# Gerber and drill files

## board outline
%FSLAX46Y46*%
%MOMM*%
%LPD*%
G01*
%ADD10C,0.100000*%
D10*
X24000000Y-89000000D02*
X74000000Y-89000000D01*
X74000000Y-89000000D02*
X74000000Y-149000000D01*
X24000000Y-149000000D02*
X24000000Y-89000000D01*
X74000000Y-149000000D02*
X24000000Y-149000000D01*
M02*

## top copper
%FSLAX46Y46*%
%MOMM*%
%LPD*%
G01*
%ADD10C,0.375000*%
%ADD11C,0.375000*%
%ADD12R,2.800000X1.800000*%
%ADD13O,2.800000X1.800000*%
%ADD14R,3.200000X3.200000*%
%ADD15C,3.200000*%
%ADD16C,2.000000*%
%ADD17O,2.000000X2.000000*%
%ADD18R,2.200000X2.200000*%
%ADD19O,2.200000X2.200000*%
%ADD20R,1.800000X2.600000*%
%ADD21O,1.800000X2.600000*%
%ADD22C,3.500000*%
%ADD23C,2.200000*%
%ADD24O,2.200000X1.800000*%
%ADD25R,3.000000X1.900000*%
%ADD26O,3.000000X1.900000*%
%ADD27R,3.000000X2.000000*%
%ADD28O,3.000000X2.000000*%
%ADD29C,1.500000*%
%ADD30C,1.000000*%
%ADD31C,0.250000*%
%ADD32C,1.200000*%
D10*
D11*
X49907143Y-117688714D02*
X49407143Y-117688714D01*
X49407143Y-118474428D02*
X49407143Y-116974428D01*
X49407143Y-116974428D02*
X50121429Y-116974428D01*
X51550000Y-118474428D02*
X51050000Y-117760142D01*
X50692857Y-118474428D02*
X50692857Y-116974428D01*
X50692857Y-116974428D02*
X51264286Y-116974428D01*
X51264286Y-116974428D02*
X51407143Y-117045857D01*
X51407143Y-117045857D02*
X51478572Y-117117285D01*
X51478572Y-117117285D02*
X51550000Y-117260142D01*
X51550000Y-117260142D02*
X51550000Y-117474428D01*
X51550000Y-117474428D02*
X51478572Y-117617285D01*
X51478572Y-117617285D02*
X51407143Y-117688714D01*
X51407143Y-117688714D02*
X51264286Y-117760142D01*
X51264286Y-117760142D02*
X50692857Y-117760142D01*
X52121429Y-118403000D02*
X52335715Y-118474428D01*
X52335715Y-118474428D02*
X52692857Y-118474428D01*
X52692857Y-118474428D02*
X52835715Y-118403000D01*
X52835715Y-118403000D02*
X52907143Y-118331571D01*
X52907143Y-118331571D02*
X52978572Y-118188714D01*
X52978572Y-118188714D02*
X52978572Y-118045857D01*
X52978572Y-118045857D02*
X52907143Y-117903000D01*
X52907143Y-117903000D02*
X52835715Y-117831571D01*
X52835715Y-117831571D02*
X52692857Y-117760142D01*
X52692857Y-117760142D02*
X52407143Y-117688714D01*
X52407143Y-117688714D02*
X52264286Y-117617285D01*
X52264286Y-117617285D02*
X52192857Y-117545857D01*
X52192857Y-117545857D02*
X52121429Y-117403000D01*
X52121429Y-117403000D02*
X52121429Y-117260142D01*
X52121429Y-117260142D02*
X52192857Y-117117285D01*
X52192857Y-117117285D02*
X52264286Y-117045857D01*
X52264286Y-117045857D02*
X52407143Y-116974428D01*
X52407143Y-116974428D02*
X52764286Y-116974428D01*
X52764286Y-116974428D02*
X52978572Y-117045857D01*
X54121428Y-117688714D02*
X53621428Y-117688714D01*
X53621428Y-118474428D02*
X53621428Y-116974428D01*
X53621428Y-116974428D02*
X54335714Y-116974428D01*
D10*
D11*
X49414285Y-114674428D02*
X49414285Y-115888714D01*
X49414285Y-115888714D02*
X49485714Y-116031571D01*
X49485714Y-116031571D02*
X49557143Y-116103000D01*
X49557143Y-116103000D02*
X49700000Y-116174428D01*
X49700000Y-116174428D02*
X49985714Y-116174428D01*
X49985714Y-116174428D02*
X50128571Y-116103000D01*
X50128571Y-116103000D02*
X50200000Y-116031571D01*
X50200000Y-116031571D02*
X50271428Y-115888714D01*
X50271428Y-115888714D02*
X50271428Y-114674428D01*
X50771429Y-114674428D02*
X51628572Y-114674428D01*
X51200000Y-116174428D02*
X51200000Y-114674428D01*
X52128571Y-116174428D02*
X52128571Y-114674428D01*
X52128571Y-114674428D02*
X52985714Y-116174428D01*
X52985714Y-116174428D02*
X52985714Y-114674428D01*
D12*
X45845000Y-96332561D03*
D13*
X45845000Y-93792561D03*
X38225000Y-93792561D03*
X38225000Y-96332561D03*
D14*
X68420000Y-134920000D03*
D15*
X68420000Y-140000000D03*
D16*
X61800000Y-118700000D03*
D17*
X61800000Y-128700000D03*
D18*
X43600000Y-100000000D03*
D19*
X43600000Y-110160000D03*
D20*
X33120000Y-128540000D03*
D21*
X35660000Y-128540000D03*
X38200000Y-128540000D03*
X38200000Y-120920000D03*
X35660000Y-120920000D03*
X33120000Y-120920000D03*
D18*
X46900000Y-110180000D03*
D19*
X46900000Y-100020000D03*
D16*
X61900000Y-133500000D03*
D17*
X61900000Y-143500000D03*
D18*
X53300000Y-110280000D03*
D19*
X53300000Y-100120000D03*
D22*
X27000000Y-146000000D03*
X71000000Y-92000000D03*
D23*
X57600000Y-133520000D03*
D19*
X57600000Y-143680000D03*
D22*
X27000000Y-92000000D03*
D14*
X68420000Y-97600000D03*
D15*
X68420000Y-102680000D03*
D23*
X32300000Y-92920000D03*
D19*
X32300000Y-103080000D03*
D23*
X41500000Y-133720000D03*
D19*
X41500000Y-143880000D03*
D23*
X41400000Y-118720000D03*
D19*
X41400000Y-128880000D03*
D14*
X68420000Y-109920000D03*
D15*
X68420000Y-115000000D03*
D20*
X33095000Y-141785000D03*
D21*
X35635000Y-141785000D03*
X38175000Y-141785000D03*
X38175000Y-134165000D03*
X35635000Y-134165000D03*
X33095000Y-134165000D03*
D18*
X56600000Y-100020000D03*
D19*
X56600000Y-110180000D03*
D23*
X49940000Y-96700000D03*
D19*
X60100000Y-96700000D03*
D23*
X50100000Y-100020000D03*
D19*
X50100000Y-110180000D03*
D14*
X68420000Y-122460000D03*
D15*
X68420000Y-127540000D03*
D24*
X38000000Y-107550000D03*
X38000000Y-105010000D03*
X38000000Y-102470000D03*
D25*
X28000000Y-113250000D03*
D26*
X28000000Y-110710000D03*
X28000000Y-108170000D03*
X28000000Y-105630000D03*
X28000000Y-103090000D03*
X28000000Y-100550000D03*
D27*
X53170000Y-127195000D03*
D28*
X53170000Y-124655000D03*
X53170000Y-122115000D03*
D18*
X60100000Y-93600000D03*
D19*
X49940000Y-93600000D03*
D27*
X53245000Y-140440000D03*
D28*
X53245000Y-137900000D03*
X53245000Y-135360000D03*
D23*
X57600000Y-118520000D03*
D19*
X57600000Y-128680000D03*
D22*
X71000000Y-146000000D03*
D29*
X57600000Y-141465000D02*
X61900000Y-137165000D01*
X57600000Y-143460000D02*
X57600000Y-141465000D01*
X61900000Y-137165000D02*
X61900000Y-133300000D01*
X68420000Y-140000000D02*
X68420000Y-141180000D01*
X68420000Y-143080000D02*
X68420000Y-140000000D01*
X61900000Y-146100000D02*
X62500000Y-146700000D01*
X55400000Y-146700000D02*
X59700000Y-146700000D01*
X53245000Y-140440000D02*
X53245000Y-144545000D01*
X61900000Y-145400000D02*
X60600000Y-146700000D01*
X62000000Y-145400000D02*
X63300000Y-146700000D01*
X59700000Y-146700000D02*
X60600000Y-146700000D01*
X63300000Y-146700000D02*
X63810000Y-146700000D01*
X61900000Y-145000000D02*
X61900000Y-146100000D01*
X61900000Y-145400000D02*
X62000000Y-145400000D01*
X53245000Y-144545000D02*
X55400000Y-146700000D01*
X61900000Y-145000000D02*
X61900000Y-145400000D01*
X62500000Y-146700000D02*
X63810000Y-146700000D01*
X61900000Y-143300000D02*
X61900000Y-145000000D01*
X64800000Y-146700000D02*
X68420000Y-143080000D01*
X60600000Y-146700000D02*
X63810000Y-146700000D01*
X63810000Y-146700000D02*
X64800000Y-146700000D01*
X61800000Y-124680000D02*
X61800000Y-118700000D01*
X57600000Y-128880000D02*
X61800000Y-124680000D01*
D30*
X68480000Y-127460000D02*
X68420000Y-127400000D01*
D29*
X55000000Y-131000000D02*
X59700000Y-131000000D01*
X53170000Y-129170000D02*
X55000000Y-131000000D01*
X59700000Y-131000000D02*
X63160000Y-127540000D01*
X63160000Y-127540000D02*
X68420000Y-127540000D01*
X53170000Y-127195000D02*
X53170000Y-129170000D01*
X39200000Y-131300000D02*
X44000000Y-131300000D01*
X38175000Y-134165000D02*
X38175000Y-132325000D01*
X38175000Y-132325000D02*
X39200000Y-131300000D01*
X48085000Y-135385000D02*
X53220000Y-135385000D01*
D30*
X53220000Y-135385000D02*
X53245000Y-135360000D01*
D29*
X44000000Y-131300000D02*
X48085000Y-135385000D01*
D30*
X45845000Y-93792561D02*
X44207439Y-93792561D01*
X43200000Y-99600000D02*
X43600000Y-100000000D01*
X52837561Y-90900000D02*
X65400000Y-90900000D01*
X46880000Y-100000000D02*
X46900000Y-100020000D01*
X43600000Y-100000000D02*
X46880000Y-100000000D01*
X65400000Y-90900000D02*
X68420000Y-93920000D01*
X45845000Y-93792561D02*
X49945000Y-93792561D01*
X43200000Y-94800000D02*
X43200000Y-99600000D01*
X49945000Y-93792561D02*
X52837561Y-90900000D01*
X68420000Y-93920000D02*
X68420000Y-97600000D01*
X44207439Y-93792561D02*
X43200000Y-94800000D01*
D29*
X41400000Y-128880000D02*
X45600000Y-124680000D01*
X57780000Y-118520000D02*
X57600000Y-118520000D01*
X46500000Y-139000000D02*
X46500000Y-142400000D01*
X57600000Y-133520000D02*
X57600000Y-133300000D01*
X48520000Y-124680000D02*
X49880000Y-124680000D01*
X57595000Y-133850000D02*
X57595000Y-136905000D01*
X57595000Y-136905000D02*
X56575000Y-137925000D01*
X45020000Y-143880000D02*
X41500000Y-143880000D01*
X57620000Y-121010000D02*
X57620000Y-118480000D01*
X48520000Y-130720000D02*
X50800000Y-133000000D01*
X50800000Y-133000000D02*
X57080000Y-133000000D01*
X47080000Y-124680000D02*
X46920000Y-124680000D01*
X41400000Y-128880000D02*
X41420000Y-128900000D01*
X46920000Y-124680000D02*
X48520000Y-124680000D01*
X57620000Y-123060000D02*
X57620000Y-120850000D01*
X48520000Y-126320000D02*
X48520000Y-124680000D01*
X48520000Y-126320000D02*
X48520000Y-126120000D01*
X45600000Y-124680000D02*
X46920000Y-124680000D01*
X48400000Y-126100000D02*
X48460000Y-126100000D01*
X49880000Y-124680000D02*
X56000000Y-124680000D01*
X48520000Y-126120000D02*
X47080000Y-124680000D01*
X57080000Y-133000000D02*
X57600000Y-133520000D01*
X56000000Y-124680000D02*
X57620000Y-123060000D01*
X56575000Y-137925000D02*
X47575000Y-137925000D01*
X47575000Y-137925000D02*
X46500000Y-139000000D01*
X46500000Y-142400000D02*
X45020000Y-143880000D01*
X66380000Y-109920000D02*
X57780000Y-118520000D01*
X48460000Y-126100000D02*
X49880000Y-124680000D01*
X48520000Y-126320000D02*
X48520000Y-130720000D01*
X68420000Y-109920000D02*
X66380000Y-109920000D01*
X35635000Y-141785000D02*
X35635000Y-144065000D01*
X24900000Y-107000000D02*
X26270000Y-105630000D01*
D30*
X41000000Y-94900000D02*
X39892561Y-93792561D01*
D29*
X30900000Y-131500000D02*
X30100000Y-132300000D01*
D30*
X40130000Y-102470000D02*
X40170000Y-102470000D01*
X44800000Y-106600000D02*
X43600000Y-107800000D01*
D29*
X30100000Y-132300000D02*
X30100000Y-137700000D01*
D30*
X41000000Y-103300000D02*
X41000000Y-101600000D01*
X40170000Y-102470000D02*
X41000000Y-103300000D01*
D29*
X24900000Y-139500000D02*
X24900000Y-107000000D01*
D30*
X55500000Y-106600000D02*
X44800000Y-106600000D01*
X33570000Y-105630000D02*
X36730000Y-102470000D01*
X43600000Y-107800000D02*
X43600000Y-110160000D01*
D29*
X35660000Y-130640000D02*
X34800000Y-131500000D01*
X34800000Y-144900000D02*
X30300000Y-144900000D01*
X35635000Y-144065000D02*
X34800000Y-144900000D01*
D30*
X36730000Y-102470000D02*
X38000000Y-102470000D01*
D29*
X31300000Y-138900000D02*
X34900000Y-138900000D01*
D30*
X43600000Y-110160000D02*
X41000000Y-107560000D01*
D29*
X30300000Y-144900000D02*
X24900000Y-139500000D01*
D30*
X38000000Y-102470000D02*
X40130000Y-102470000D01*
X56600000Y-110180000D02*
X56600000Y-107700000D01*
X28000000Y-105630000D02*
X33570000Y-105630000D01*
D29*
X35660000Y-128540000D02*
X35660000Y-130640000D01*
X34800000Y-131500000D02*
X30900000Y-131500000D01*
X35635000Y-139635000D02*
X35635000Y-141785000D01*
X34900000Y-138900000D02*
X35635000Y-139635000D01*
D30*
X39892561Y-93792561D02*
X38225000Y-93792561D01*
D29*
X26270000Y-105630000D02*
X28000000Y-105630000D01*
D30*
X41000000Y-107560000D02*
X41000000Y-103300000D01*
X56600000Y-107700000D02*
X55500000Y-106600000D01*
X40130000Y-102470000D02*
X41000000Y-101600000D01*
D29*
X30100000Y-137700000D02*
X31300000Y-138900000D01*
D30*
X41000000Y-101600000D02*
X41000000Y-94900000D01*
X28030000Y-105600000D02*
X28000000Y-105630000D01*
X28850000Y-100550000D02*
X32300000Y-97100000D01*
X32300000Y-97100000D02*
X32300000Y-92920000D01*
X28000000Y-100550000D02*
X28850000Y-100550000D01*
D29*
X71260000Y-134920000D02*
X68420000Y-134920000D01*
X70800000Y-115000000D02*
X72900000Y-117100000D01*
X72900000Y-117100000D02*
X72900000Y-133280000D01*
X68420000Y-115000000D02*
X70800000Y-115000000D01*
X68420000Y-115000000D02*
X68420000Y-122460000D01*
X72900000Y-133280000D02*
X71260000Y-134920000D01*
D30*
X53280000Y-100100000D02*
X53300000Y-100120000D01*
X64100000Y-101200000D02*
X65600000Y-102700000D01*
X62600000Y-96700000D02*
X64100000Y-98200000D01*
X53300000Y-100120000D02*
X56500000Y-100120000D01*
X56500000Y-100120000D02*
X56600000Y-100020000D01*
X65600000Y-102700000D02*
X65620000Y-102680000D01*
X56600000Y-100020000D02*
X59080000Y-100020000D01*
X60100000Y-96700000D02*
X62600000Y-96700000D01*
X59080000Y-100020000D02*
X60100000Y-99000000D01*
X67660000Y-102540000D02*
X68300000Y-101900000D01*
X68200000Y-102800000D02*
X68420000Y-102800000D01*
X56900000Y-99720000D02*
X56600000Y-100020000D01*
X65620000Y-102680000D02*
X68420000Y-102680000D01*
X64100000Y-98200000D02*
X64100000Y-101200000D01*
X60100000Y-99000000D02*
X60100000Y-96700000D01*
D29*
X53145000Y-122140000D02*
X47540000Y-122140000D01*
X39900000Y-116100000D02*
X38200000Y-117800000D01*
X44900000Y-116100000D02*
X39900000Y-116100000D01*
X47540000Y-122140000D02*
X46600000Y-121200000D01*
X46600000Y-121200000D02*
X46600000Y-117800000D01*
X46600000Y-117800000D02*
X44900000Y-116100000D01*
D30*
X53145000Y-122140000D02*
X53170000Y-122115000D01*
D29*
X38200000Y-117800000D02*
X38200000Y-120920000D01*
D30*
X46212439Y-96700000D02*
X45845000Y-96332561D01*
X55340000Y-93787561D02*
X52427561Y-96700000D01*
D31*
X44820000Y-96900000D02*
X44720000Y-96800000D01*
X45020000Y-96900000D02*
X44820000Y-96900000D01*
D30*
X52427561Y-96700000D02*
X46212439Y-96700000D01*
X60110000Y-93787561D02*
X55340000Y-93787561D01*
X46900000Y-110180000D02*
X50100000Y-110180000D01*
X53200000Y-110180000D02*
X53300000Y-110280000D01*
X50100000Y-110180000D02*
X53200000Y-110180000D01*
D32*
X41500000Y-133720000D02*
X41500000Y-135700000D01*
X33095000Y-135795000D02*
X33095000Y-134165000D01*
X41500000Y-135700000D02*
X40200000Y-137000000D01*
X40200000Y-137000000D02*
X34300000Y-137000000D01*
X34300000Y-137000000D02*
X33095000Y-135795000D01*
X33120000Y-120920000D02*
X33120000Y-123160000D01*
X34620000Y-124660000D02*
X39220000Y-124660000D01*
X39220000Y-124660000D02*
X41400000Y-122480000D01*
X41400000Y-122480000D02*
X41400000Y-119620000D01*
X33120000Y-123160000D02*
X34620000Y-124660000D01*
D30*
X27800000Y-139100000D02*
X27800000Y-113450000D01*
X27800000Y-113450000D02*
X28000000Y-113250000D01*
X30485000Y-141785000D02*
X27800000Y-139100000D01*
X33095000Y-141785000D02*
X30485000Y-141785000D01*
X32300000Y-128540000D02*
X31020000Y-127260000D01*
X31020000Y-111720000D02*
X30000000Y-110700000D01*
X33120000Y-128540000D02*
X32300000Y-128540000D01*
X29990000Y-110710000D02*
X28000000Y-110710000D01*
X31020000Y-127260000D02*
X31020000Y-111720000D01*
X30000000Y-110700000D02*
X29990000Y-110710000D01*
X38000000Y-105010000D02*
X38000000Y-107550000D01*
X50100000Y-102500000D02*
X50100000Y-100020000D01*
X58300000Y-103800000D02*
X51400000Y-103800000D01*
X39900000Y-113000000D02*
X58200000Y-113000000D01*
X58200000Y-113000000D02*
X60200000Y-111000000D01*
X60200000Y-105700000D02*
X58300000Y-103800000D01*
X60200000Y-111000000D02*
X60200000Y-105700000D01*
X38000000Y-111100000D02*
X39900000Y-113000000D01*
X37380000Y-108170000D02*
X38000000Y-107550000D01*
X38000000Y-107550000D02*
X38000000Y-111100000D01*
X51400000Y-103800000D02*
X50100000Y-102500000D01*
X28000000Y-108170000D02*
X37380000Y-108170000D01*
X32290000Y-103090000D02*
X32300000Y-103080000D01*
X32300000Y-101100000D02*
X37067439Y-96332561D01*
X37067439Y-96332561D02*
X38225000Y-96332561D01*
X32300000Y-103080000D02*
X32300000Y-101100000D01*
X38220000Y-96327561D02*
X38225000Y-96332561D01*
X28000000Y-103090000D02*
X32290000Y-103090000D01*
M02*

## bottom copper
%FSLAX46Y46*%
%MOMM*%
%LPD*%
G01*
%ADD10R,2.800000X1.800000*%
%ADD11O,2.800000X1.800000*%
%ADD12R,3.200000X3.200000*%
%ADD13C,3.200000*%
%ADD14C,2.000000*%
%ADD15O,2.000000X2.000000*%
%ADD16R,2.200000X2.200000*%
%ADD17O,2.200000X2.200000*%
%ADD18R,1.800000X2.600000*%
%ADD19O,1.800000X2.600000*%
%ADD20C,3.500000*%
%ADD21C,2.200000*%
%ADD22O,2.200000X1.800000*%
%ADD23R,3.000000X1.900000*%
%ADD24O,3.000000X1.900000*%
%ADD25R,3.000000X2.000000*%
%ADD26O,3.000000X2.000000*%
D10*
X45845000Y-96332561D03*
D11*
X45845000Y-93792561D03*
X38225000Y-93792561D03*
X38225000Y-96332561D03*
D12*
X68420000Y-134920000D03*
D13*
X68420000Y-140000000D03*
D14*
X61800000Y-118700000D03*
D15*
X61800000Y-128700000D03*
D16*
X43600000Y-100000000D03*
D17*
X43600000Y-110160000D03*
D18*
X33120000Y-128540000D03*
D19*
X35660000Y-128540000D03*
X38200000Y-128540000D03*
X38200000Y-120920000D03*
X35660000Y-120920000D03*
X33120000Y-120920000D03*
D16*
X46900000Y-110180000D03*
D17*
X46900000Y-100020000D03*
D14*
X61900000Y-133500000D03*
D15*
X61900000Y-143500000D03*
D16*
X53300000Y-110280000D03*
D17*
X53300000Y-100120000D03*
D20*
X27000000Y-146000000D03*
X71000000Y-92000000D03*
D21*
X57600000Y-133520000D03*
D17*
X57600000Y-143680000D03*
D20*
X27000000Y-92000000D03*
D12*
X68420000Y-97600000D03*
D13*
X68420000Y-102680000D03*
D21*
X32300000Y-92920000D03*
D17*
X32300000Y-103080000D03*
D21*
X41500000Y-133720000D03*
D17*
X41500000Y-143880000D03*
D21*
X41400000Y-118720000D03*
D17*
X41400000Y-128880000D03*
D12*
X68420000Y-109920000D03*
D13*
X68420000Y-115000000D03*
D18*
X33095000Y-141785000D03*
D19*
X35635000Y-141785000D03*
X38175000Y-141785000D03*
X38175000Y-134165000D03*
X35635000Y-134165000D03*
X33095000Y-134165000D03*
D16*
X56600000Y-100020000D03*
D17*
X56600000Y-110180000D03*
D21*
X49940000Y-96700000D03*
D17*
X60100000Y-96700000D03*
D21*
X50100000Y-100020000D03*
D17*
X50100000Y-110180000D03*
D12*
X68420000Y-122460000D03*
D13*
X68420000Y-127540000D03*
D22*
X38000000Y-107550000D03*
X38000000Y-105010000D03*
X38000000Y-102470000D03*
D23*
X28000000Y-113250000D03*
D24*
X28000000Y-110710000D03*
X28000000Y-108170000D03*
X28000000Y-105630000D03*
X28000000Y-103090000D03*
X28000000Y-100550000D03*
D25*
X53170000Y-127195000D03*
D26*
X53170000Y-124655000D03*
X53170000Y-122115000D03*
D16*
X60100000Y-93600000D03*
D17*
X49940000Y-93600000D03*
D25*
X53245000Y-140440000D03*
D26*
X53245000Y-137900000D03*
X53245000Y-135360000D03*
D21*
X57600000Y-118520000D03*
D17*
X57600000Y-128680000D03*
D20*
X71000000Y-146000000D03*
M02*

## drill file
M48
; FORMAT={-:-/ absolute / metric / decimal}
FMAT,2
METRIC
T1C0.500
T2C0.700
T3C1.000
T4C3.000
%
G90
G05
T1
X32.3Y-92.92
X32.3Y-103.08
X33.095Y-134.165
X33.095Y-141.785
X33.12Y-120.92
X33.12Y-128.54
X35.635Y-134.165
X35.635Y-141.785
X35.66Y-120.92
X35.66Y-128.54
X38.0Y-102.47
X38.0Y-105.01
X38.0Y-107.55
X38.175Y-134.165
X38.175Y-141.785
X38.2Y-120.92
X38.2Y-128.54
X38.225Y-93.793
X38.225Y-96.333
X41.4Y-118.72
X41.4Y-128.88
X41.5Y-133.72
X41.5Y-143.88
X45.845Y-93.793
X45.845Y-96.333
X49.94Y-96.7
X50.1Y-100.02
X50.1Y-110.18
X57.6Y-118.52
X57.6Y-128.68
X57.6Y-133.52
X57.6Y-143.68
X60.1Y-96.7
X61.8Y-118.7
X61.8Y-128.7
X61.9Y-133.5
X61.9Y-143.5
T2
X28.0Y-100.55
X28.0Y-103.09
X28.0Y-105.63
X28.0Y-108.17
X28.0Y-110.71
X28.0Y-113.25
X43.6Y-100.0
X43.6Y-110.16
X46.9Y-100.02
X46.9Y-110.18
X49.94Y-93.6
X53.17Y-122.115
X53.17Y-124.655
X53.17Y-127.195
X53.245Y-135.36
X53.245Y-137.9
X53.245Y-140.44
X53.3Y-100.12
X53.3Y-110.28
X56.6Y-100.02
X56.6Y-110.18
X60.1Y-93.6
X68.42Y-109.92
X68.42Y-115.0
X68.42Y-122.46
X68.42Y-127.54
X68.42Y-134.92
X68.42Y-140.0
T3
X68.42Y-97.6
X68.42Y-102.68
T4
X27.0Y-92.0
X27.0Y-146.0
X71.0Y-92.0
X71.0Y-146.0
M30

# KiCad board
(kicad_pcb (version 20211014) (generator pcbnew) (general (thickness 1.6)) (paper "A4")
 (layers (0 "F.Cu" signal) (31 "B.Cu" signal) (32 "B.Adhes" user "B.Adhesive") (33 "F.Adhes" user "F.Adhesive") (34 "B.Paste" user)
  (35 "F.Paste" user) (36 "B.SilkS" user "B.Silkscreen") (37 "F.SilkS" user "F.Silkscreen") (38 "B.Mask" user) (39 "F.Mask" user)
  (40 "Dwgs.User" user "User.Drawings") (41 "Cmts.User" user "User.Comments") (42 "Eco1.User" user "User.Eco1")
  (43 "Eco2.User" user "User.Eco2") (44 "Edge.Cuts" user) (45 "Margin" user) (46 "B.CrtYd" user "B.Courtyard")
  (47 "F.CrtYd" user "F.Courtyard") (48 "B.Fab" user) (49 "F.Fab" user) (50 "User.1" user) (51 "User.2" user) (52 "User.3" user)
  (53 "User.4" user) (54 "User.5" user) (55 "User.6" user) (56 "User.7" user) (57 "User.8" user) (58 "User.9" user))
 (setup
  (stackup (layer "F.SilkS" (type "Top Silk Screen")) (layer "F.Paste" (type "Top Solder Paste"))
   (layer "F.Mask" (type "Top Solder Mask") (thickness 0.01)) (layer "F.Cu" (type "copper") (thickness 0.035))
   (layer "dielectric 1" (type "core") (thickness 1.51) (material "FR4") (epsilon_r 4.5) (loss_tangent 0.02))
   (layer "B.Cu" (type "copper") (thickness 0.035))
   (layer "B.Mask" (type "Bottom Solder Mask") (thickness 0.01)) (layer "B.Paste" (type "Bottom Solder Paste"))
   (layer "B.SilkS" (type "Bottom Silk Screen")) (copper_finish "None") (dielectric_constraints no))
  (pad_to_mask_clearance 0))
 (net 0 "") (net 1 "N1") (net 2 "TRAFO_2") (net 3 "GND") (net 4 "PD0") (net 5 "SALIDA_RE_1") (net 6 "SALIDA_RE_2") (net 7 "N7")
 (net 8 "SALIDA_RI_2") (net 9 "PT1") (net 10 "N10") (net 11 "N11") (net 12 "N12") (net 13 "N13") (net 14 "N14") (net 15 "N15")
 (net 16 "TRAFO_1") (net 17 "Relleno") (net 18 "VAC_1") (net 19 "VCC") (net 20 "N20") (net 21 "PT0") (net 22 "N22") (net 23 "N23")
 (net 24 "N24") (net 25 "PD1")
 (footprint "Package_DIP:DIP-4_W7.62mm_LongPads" (layer "F.Cu") (at 45.845 96.332561 180)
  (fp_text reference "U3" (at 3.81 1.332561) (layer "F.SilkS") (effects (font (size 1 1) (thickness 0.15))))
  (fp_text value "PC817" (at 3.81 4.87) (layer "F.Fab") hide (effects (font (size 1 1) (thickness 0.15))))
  (pad "1" thru_hole rect (at 0 0 180) (size 2.8 1.8) (drill 0.5) (layers *.Cu *.Mask) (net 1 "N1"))
  (pad "2" thru_hole oval (at 0 2.54 180) (size 2.8 1.8) (drill 0.5) (layers *.Cu *.Mask) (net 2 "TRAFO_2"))
  (pad "3" thru_hole oval (at 7.62 2.54 180) (size 2.8 1.8) (drill 0.5) (layers *.Cu *.Mask) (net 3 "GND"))
  (pad "4" thru_hole oval (at 7.62 0 180) (size 2.8 1.8) (drill 0.5) (layers *.Cu *.Mask) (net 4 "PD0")))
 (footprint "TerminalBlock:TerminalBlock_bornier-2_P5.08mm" (layer "F.Cu") (at 68.42 134.92 -90)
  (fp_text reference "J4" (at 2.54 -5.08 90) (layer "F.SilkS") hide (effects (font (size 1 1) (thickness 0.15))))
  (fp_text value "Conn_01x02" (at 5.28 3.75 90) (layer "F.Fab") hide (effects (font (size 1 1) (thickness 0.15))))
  (pad "1" thru_hole rect (at 0 0 270) (size 3.2 3.2) (drill 0.7) (layers *.Cu *.Mask) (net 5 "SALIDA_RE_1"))
  (pad "2" thru_hole circle (at 5.08 0 270) (size 3.2 3.2) (drill 0.7) (layers *.Cu *.Mask) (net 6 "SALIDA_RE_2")))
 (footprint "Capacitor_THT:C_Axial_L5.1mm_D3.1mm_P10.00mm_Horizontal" (layer "F.Cu") (at 61.8 118.7 -90)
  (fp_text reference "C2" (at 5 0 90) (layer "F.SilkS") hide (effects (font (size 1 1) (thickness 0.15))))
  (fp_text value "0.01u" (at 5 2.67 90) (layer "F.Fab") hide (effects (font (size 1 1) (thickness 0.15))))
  (pad "1" thru_hole circle (at 0 0 270) (size 2 2) (drill 0.5) (layers *.Cu *.Mask) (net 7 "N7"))
  (pad "2" thru_hole oval (at 10 0 270) (size 2 2) (drill 0.5) (layers *.Cu *.Mask) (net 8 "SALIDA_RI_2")))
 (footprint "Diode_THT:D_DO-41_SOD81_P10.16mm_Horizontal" (layer "F.Cu") (at 43.6 100 -90)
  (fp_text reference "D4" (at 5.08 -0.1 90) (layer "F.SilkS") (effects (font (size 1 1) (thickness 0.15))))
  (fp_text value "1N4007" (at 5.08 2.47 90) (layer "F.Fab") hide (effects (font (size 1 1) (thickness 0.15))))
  (pad "1" thru_hole rect (at 0 0 270) (size 2.2 2.2) (drill 0.7) (layers *.Cu *.Mask) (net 2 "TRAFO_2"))
  (pad "2" thru_hole oval (at 10.16 0 270) (size 2.2 2.2) (drill 0.7) (layers *.Cu *.Mask) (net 3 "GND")))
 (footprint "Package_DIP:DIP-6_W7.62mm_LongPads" (layer "F.Cu") (at 33.12 128.54 90)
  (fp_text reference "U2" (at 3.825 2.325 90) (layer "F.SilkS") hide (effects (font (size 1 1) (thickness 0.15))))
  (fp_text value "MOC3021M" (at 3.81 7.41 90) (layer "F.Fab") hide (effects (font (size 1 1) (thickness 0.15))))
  (pad "1" thru_hole rect (at 0 0 90) (size 2.6 1.8) (drill 0.5) (layers *.Cu *.Mask) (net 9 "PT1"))
  (pad "2" thru_hole oval (at 0 2.54 90) (size 2.6 1.8) (drill 0.5) (layers *.Cu *.Mask) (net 3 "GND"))
  (pad "3" thru_hole oval (at 0 5.08 90) (size 2.6 1.8) (drill 0.5) (layers *.Cu *.Mask) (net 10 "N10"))
  (pad "4" thru_hole oval (at 7.62 5.08 90) (size 2.6 1.8) (drill 0.5) (layers *.Cu *.Mask) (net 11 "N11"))
  (pad "5" thru_hole oval (at 7.62 2.54 90) (size 2.6 1.8) (drill 0.5) (layers *.Cu *.Mask) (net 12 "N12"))
  (pad "6" thru_hole oval (at 7.62 0 90) (size 2.6 1.8) (drill 0.5) (layers *.Cu *.Mask) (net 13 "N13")))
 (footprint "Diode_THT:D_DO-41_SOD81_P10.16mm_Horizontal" (layer "F.Cu") (at 46.9 110.18 90)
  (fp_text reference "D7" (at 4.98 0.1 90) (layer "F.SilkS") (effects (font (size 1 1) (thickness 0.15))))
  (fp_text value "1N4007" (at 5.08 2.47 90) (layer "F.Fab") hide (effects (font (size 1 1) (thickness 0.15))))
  (pad "1" thru_hole rect (at 0 0 90) (size 2.2 2.2) (drill 0.7) (layers *.Cu *.Mask) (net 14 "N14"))
  (pad "2" thru_hole oval (at 10.16 0 90) (size 2.2 2.2) (drill 0.7) (layers *.Cu *.Mask) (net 2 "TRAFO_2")))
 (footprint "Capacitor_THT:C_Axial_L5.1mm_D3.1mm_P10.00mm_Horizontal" (layer "F.Cu") (at 61.9 133.5 -90)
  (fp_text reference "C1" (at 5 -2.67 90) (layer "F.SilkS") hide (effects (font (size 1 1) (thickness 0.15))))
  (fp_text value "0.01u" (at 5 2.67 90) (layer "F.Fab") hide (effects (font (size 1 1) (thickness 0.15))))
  (pad "1" thru_hole circle (at 0 0 270) (size 2 2) (drill 0.5) (layers *.Cu *.Mask) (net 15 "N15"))
  (pad "2" thru_hole oval (at 10 0 270) (size 2 2) (drill 0.5) (layers *.Cu *.Mask) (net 6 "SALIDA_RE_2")))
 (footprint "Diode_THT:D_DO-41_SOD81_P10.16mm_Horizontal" (layer "F.Cu") (at 53.3 110.28 90)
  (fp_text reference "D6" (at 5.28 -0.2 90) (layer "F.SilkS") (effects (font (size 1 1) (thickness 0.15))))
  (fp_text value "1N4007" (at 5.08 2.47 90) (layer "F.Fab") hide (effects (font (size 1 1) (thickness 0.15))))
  (pad "1" thru_hole rect (at 0 0 90) (size 2.2 2.2) (drill 0.7) (layers *.Cu *.Mask) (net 14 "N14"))
  (pad "2" thru_hole oval (at 10.16 0 90) (size 2.2 2.2) (drill 0.7) (layers *.Cu *.Mask) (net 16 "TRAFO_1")))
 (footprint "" (layer "F.Cu") (at 27 146)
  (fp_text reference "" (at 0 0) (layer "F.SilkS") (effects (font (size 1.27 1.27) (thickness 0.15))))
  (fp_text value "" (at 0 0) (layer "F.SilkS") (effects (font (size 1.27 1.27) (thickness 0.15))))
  (pad "1" thru_hole circle (at 0 0) (size 3.5 3.5) (drill 3) (layers *.Cu *.Mask) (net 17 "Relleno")))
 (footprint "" (layer "F.Cu") (at 71 92)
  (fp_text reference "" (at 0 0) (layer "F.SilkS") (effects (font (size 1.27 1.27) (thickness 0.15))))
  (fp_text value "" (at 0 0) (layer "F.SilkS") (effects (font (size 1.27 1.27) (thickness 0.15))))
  (pad "1" thru_hole circle (at 0 0) (size 3.5 3.5) (drill 3) (layers *.Cu *.Mask) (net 17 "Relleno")))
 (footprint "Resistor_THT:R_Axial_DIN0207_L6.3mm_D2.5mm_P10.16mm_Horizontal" (layer "F.Cu") (at 57.6 133.52 -90)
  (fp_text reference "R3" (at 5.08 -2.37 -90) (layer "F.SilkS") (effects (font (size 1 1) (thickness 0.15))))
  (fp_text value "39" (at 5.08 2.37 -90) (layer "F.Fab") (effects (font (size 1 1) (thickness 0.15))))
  (pad "1" thru_hole circle (at 0 0 270) (size 2.2 2.2) (drill 0.5) (layers *.Cu *.Mask) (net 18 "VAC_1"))
  (pad "2" thru_hole oval (at 10.16 0 270) (size 2.2 2.2) (drill 0.5) (layers *.Cu *.Mask) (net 15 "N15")))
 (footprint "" (layer "F.Cu") (at 27 92)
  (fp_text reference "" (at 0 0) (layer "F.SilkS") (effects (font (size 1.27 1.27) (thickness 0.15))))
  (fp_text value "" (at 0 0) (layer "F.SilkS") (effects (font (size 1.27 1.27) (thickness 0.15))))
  (pad "1" thru_hole circle (at 0 0) (size 3.5 3.5) (drill 3) (layers *.Cu *.Mask) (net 17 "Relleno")))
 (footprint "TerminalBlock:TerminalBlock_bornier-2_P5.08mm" (layer "F.Cu") (at 68.42 97.6 -90)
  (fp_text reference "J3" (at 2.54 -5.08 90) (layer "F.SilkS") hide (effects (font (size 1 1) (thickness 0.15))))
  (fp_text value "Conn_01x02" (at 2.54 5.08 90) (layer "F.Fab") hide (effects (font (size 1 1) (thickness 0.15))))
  (pad "1" thru_hole rect (at 0 0 270) (size 3.2 3.2) (drill 1) (layers *.Cu *.Mask) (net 2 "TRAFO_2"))
  (pad "2" thru_hole circle (at 5.08 0 270) (size 3.2 3.2) (drill 1) (layers *.Cu *.Mask) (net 16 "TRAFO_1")))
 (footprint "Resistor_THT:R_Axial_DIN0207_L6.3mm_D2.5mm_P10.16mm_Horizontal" (layer "F.Cu") (at 32.3 92.92 -90)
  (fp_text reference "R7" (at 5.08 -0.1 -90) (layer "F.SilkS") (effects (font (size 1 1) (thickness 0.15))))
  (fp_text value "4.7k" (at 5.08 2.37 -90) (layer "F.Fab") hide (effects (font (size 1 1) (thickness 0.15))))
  (pad "1" thru_hole circle (at 0 0 270) (size 2.2 2.2) (drill 0.5) (layers *.Cu *.Mask) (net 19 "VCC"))
  (pad "2" thru_hole oval (at 10.16 0 270) (size 2.2 2.2) (drill 0.5) (layers *.Cu *.Mask) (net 4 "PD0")))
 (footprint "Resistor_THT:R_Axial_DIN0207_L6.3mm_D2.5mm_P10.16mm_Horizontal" (layer "F.Cu") (at 41.5 133.72 -90)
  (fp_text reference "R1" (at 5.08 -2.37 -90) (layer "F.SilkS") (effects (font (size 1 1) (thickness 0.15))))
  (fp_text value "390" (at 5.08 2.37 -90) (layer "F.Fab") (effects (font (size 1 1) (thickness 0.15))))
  (pad "1" thru_hole circle (at 0 0 270) (size 2.2 2.2) (drill 0.5) (layers *.Cu *.Mask) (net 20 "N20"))
  (pad "2" thru_hole oval (at 10.16 0 270) (size 2.2 2.2) (drill 0.5) (layers *.Cu *.Mask) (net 18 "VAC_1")))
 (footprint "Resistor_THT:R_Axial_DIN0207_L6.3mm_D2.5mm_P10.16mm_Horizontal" (layer "F.Cu") (at 41.4 118.72 -90)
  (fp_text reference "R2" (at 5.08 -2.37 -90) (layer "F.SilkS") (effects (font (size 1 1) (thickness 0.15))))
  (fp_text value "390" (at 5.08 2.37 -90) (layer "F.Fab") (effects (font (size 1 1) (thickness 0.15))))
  (pad "1" thru_hole circle (at 0 0 270) (size 2.2 2.2) (drill 0.5) (layers *.Cu *.Mask) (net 13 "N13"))
  (pad "2" thru_hole oval (at 10.16 0 270) (size 2.2 2.2) (drill 0.5) (layers *.Cu *.Mask) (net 18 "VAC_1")))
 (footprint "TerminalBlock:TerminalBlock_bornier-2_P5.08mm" (layer "F.Cu") (at 68.42 109.92 -90)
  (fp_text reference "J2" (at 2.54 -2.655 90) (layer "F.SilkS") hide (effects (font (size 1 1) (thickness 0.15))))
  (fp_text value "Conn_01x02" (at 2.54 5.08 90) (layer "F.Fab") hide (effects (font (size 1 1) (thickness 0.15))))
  (pad "1" thru_hole rect (at 0 0 270) (size 3.2 3.2) (drill 0.7) (layers *.Cu *.Mask) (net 18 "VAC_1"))
  (pad "2" thru_hole circle (at 5.08 0 270) (size 3.2 3.2) (drill 0.7) (layers *.Cu *.Mask) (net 5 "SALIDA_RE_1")))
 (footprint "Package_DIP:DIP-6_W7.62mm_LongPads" (layer "F.Cu") (at 33.095 141.785 90)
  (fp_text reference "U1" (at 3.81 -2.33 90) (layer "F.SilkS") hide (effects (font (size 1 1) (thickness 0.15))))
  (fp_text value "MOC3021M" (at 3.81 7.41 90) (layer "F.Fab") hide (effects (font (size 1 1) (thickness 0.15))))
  (pad "1" thru_hole rect (at 0 0 90) (size 2.6 1.8) (drill 0.5) (layers *.Cu *.Mask) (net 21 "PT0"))
  (pad "2" thru_hole oval (at 0 2.54 90) (size 2.6 1.8) (drill 0.5) (layers *.Cu *.Mask) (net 3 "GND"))
  (pad "3" thru_hole oval (at 0 5.08 90) (size 2.6 1.8) (drill 0.5) (layers *.Cu *.Mask) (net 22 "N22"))
  (pad "4" thru_hole oval (at 7.62 5.08 90) (size 2.6 1.8) (drill 0.5) (layers *.Cu *.Mask) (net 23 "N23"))
  (pad "5" thru_hole oval (at 7.62 2.54 90) (size 2.6 1.8) (drill 0.5) (layers *.Cu *.Mask) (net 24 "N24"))
  (pad "6" thru_hole oval (at 7.62 0 90) (size 2.6 1.8) (drill 0.5) (layers *.Cu *.Mask) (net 20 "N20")))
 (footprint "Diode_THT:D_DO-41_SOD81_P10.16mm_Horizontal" (layer "F.Cu") (at 56.6 100.02 -90)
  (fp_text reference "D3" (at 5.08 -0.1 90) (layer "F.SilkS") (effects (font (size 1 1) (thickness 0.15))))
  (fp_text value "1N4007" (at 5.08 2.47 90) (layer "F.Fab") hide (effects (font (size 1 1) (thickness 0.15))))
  (pad "1" thru_hole rect (at 0 0 270) (size 2.2 2.2) (drill 0.7) (layers *.Cu *.Mask) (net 16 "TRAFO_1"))
  (pad "2" thru_hole oval (at 10.16 0 270) (size 2.2 2.2) (drill 0.7) (layers *.Cu *.Mask) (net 3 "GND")))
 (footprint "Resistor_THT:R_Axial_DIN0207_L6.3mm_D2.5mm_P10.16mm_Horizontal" (layer "F.Cu") (at 49.94 96.7)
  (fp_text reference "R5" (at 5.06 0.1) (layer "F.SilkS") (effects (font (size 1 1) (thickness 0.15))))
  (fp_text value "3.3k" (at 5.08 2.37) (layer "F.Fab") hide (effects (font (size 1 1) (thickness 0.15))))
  (pad "1" thru_hole circle (at 0 0) (size 2.2 2.2) (drill 0.5) (layers *.Cu *.Mask) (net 1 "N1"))
  (pad "2" thru_hole oval (at 10.16 0) (size 2.2 2.2) (drill 0.5) (layers *.Cu *.Mask) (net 16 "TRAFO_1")))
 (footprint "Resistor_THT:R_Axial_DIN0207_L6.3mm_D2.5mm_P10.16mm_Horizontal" (layer "F.Cu") (at 50.1 100.02 -90)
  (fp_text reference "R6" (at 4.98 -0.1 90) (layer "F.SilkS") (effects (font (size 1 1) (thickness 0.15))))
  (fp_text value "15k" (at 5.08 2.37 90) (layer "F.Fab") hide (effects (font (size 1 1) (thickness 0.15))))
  (pad "1" thru_hole circle (at 0 0 270) (size 2.2 2.2) (drill 0.5) (layers *.Cu *.Mask) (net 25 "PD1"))
  (pad "2" thru_hole oval (at 10.16 0 270) (size 2.2 2.2) (drill 0.5) (layers *.Cu *.Mask) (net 14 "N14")))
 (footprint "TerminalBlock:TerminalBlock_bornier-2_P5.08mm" (layer "F.Cu") (at 68.42 122.46 -90)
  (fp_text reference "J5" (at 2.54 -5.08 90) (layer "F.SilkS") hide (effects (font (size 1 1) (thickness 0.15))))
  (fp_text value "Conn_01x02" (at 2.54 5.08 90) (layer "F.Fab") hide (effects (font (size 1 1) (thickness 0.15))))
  (pad "1" thru_hole rect (at 0 0 270) (size 3.2 3.2) (drill 0.7) (layers *.Cu *.Mask) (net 5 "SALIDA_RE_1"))
  (pad "2" thru_hole circle (at 5.08 0 270) (size 3.2 3.2) (drill 0.7) (layers *.Cu *.Mask) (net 8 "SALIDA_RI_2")))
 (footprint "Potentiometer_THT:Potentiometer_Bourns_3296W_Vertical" (layer "F.Cu") (at 38 107.55 -90)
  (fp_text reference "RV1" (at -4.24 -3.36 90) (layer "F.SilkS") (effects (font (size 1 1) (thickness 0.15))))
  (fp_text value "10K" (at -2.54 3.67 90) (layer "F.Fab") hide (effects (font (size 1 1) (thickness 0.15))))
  (pad "1" thru_hole oval (at 0 0 270) (size 1.8 2.2) (drill 0.5) (layers *.Cu *.Mask) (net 25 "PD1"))
  (pad "2" thru_hole oval (at -2.54 0 270) (size 1.8 2.2) (drill 0.5) (layers *.Cu *.Mask) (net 25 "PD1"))
  (pad "3" thru_hole oval (at -5.08 0 270) (size 1.8 2.2) (drill 0.5) (layers *.Cu *.Mask) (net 3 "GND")))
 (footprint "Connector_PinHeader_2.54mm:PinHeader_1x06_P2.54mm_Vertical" (layer "F.Cu") (at 28 113.25 180)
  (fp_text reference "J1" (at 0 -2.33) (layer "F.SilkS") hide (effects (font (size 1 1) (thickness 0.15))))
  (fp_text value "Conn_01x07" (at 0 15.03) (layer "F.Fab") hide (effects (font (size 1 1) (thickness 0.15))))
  (pad "1" thru_hole rect (at 0 0 180) (size 3 1.9) (drill 0.7) (layers *.Cu *.Mask) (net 21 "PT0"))
  (pad "2" thru_hole oval (at 0 2.54 180) (size 3 1.9) (drill 0.7) (layers *.Cu *.Mask) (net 9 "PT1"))
  (pad "3" thru_hole oval (at 0 5.08 180) (size 3 1.9) (drill 0.7) (layers *.Cu *.Mask) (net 25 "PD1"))
  (pad "4" thru_hole oval (at 0 7.62 180) (size 3 1.9) (drill 0.7) (layers *.Cu *.Mask) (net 3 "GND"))
  (pad "5" thru_hole oval (at 0 10.16 180) (size 3 1.9) (drill 0.7) (layers *.Cu *.Mask) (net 4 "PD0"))
  (pad "6" thru_hole oval (at 0 12.7 180) (size 3 1.9) (drill 0.7) (layers *.Cu *.Mask) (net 19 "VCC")))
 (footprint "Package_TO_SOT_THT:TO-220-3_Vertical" (layer "F.Cu") (at 53.17 127.195 90)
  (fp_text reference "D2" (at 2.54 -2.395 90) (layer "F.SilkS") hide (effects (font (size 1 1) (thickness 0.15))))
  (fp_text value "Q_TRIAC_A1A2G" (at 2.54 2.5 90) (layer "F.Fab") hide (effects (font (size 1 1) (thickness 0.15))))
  (pad "1" thru_hole rect (at 0 0 90) (size 2 3) (drill 0.7) (layers *.Cu *.Mask) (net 8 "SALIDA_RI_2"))
  (pad "2" thru_hole oval (at 2.54 0 90) (size 2 3) (drill 0.7) (layers *.Cu *.Mask) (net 18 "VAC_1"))
  (pad "3" thru_hole oval (at 5.08 0 90) (size 2 3) (drill 0.7) (layers *.Cu *.Mask) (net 11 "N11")))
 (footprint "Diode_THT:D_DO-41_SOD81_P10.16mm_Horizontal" (layer "F.Cu") (at 60.1 93.6 180)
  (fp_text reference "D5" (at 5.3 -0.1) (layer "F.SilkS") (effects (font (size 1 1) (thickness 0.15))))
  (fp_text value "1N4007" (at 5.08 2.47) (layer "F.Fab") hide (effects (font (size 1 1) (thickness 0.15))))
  (pad "1" thru_hole rect (at 0 0 180) (size 2.2 2.2) (drill 0.7) (layers *.Cu *.Mask) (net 1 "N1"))
  (pad "2" thru_hole oval (at 10.16 0 180) (size 2.2 2.2) (drill 0.7) (layers *.Cu *.Mask) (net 2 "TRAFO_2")))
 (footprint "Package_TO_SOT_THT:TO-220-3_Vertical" (layer "F.Cu") (at 53.245 140.44 90)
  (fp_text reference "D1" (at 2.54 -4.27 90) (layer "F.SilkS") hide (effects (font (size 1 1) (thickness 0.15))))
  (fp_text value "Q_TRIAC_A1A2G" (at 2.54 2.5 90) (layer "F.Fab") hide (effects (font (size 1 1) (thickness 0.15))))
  (pad "1" thru_hole rect (at 0 0 90) (size 2 3) (drill 0.7) (layers *.Cu *.Mask) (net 6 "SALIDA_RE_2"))
  (pad "2" thru_hole oval (at 2.54 0 90) (size 2 3) (drill 0.7) (layers *.Cu *.Mask) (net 18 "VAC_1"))
  (pad "3" thru_hole oval (at 5.08 0 90) (size 2 3) (drill 0.7) (layers *.Cu *.Mask) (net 23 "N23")))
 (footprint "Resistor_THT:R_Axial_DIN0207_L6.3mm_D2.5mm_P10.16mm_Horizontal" (layer "F.Cu") (at 57.6 118.52 -90)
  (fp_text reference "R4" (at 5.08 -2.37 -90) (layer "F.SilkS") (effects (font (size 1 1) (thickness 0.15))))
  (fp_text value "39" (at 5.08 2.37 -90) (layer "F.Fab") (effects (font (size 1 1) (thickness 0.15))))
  (pad "1" thru_hole circle (at 0 0 270) (size 2.2 2.2) (drill 0.5) (layers *.Cu *.Mask) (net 18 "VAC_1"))
  (pad "2" thru_hole oval (at 10.16 0 270) (size 2.2 2.2) (drill 0.5) (layers *.Cu *.Mask) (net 7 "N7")))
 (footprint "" (layer "F.Cu") (at 71 146)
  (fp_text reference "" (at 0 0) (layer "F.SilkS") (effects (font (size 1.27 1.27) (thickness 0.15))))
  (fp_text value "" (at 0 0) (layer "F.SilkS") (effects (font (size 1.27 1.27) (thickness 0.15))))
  (pad "1" thru_hole circle (at 0 0) (size 3.5 3.5) (drill 3) (layers *.Cu *.Mask) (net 17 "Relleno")))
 (gr_line (start 24 89) (end 74 89) (layer "Edge.Cuts") (width 0.1))
 (gr_line (start 74 89) (end 74 149) (layer "Edge.Cuts") (width 0.1))
 (gr_line (start 24 149) (end 24 89) (layer "Edge.Cuts") (width 0.1))
 (gr_line (start 74 149) (end 24 149) (layer "Edge.Cuts") (width 0.1))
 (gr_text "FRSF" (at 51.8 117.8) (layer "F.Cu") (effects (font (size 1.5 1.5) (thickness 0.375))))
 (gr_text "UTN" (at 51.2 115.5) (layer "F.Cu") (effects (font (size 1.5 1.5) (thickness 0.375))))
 (segment (start 57.6 141.465) (end 61.9 137.165) (width 1.5) (layer "F.Cu") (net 15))
 (segment (start 57.6 143.46) (end 57.6 141.465) (width 1.5) (layer "F.Cu") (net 15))
 (segment (start 61.9 137.165) (end 61.9 133.3) (width 1.5) (layer "F.Cu") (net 15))
 (segment (start 68.42 140) (end 68.42 141.18) (width 1.5) (layer "F.Cu") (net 6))
 (segment (start 68.42 143.08) (end 68.42 140) (width 1.5) (layer "F.Cu") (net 6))
 (segment (start 61.9 146.1) (end 62.5 146.7) (width 1.5) (layer "F.Cu") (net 6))
 (segment (start 55.4 146.7) (end 59.7 146.7) (width 1.5) (layer "F.Cu") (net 6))
 (segment (start 53.245 140.44) (end 53.245 144.545) (width 1.5) (layer "F.Cu") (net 6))
 (segment (start 61.9 145.4) (end 60.6 146.7) (width 1.5) (layer "F.Cu") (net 6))
 (segment (start 62 145.4) (end 63.3 146.7) (width 1.5) (layer "F.Cu") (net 6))
 (segment (start 59.7 146.7) (end 60.6 146.7) (width 1.5) (layer "F.Cu") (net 6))
 (segment (start 63.3 146.7) (end 63.81 146.7) (width 1.5) (layer "F.Cu") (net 6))
 (segment (start 61.9 145) (end 61.9 146.1) (width 1.5) (layer "F.Cu") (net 6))
 (segment (start 61.9 145.4) (end 62 145.4) (width 1.5) (layer "F.Cu") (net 6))
 (segment (start 53.245 144.545) (end 55.4 146.7) (width 1.5) (layer "F.Cu") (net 6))
 (segment (start 61.9 145) (end 61.9 145.4) (width 1.5) (layer "F.Cu") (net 6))
 (segment (start 62.5 146.7) (end 63.81 146.7) (width 1.5) (layer "F.Cu") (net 6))
 (segment (start 61.9 143.3) (end 61.9 145) (width 1.5) (layer "F.Cu") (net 6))
 (segment (start 64.8 146.7) (end 68.42 143.08) (width 1.5) (layer "F.Cu") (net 6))
 (segment (start 60.6 146.7) (end 63.81 146.7) (width 1.5) (layer "F.Cu") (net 6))
 (segment (start 63.81 146.7) (end 64.8 146.7) (width 1.5) (layer "F.Cu") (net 6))
 (segment (start 61.8 124.68) (end 61.8 118.7) (width 1.5) (layer "F.Cu") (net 7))
 (segment (start 57.6 128.88) (end 61.8 124.68) (width 1.5) (layer "F.Cu") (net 7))
 (segment (start 68.48 127.46) (end 68.42 127.4) (width 1) (layer "F.Cu") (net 8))
 (segment (start 55 131) (end 59.7 131) (width 1.5) (layer "F.Cu") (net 8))
 (segment (start 53.17 129.17) (end 55 131) (width 1.5) (layer "F.Cu") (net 8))
 (segment (start 59.7 131) (end 63.16 127.54) (width 1.5) (layer "F.Cu") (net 8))
 (segment (start 63.16 127.54) (end 68.42 127.54) (width 1.5) (layer "F.Cu") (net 8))
 (segment (start 53.17 127.195) (end 53.17 129.17) (width 1.5) (layer "F.Cu") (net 8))
 (segment (start 39.2 131.3) (end 44 131.3) (width 1.5) (layer "F.Cu") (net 23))
 (segment (start 38.175 134.165) (end 38.175 132.325) (width 1.5) (layer "F.Cu") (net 23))
 (segment (start 38.175 132.325) (end 39.2 131.3) (width 1.5) (layer "F.Cu") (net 23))
 (segment (start 48.085 135.385) (end 53.22 135.385) (width 1.5) (layer "F.Cu") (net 23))
 (segment (start 53.22 135.385) (end 53.245 135.36) (width 1) (layer "F.Cu") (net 23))
 (segment (start 44 131.3) (end 48.085 135.385) (width 1.5) (layer "F.Cu") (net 23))
 (segment (start 45.845 93.792561) (end 44.207439 93.792561) (width 1) (layer "F.Cu") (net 2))
 (segment (start 43.2 99.6) (end 43.6 100) (width 1) (layer "F.Cu") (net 2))
 (segment (start 52.837561 90.9) (end 65.4 90.9) (width 1) (layer "F.Cu") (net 2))
 (segment (start 46.88 100) (end 46.9 100.02) (width 1) (layer "F.Cu") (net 2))
 (segment (start 43.6 100) (end 46.88 100) (width 1) (layer "F.Cu") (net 2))
 (segment (start 65.4 90.9) (end 68.42 93.92) (width 1) (layer "F.Cu") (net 2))
 (segment (start 45.845 93.792561) (end 49.945 93.792561) (width 1) (layer "F.Cu") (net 2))
 (segment (start 43.2 94.8) (end 43.2 99.6) (width 1) (layer "F.Cu") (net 2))
 (segment (start 49.945 93.792561) (end 52.837561 90.9) (width 1) (layer "F.Cu") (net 2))
 (segment (start 68.42 93.92) (end 68.42 97.6) (width 1) (layer "F.Cu") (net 2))
 (segment (start 44.207439 93.792561) (end 43.2 94.8) (width 1) (layer "F.Cu") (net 2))
 (segment (start 41.4 128.88) (end 45.6 124.68) (width 1.5) (layer "F.Cu") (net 18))
 (segment (start 57.78 118.52) (end 57.6 118.52) (width 1.5) (layer "F.Cu") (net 18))
 (segment (start 46.5 139) (end 46.5 142.4) (width 1.5) (layer "F.Cu") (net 18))
 (segment (start 57.6 133.52) (end 57.6 133.3) (width 1.5) (layer "F.Cu") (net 18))
 (segment (start 48.52 124.68) (end 49.88 124.68) (width 1.5) (layer "F.Cu") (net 18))
 (segment (start 57.595 133.85) (end 57.595 136.905) (width 1.5) (layer "F.Cu") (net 18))
 (segment (start 57.595 136.905) (end 56.575 137.925) (width 1.5) (layer "F.Cu") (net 18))
 (segment (start 45.02 143.88) (end 41.5 143.88) (width 1.5) (layer "F.Cu") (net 18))
 (segment (start 57.62 121.01) (end 57.62 118.48) (width 1.5) (layer "F.Cu") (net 18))
 (segment (start 48.52 130.72) (end 50.8 133) (width 1.5) (layer "F.Cu") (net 18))
 (segment (start 50.8 133) (end 57.08 133) (width 1.5) (layer "F.Cu") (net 18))
 (segment (start 47.08 124.68) (end 46.92 124.68) (width 1.5) (layer "F.Cu") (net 18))
 (segment (start 41.4 128.88) (end 41.42 128.9) (width 1.5) (layer "F.Cu") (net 18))
 (segment (start 46.92 124.68) (end 48.52 124.68) (width 1.5) (layer "F.Cu") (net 18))
 (segment (start 57.62 123.06) (end 57.62 120.85) (width 1.5) (layer "F.Cu") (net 18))
 (segment (start 48.52 126.32) (end 48.52 124.68) (width 1.5) (layer "F.Cu") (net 18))
 (segment (start 48.52 126.32) (end 48.52 126.12) (width 1.5) (layer "F.Cu") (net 18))
 (segment (start 45.6 124.68) (end 46.92 124.68) (width 1.5) (layer "F.Cu") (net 18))
 (segment (start 48.4 126.1) (end 48.46 126.1) (width 1.5) (layer "F.Cu") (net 18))
 (segment (start 49.88 124.68) (end 56 124.68) (width 1.5) (layer "F.Cu") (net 18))
 (segment (start 48.52 126.12) (end 47.08 124.68) (width 1.5) (layer "F.Cu") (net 18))
 (segment (start 57.08 133) (end 57.6 133.52) (width 1.5) (layer "F.Cu") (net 18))
 (segment (start 56 124.68) (end 57.62 123.06) (width 1.5) (layer "F.Cu") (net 18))
 (segment (start 56.575 137.925) (end 47.575 137.925) (width 1.5) (layer "F.Cu") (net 18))
 (segment (start 47.575 137.925) (end 46.5 139) (width 1.5) (layer "F.Cu") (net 18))
 (segment (start 46.5 142.4) (end 45.02 143.88) (width 1.5) (layer "F.Cu") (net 18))
 (segment (start 66.38 109.92) (end 57.78 118.52) (width 1.5) (layer "F.Cu") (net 18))
 (segment (start 48.46 126.1) (end 49.88 124.68) (width 1.5) (layer "F.Cu") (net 18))
 (segment (start 48.52 126.32) (end 48.52 130.72) (width 1.5) (layer "F.Cu") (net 18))
 (segment (start 68.42 109.92) (end 66.38 109.92) (width 1.5) (layer "F.Cu") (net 18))
 (segment (start 35.635 141.785) (end 35.635 144.065) (width 1.5) (layer "F.Cu") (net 3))
 (segment (start 24.9 107) (end 26.27 105.63) (width 1.5) (layer "F.Cu") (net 3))
 (segment (start 41 94.9) (end 39.892561 93.792561) (width 1) (layer "F.Cu") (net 3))
 (segment (start 30.9 131.5) (end 30.1 132.3) (width 1.5) (layer "F.Cu") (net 3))
 (segment (start 40.13 102.47) (end 40.17 102.47) (width 1) (layer "F.Cu") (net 3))
 (segment (start 44.8 106.6) (end 43.6 107.8) (width 1) (layer "F.Cu") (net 3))
 (segment (start 30.1 132.3) (end 30.1 137.7) (width 1.5) (layer "F.Cu") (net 3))
 (segment (start 41 103.3) (end 41 101.6) (width 1) (layer "F.Cu") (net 3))
 (segment (start 40.17 102.47) (end 41 103.3) (width 1) (layer "F.Cu") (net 3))
 (segment (start 24.9 139.5) (end 24.9 107) (width 1.5) (layer "F.Cu") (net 3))
 (segment (start 55.5 106.6) (end 44.8 106.6) (width 1) (layer "F.Cu") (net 3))
 (segment (start 33.57 105.63) (end 36.73 102.47) (width 1) (layer "F.Cu") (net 3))
 (segment (start 43.6 107.8) (end 43.6 110.16) (width 1) (layer "F.Cu") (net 3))
 (segment (start 35.66 130.64) (end 34.8 131.5) (width 1.5) (layer "F.Cu") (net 3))
 (segment (start 34.8 144.9) (end 30.3 144.9) (width 1.5) (layer "F.Cu") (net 3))
 (segment (start 35.635 144.065) (end 34.8 144.9) (width 1.5) (layer "F.Cu") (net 3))
 (segment (start 36.73 102.47) (end 38 102.47) (width 1) (layer "F.Cu") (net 3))
 (segment (start 31.3 138.9) (end 34.9 138.9) (width 1.5) (layer "F.Cu") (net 3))
 (segment (start 43.6 110.16) (end 41 107.56) (width 1) (layer "F.Cu") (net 3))
 (segment (start 30.3 144.9) (end 24.9 139.5) (width 1.5) (layer "F.Cu") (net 3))
 (segment (start 38 102.47) (end 40.13 102.47) (width 1) (layer "F.Cu") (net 3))
 (segment (start 56.6 110.18) (end 56.6 107.7) (width 1) (layer "F.Cu") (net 3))
 (segment (start 28 105.63) (end 33.57 105.63) (width 1) (layer "F.Cu") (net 3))
 (segment (start 35.66 128.54) (end 35.66 130.64) (width 1.5) (layer "F.Cu") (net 3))
 (segment (start 34.8 131.5) (end 30.9 131.5) (width 1.5) (layer "F.Cu") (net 3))
 (segment (start 35.635 139.635) (end 35.635 141.785) (width 1.5) (layer "F.Cu") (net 3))
 (segment (start 34.9 138.9) (end 35.635 139.635) (width 1.5) (layer "F.Cu") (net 3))
 (segment (start 39.892561 93.792561) (end 38.225 93.792561) (width 1) (layer "F.Cu") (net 3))
 (segment (start 26.27 105.63) (end 28 105.63) (width 1.5) (layer "F.Cu") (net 3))
 (segment (start 41 107.56) (end 41 103.3) (width 1) (layer "F.Cu") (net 3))
 (segment (start 56.6 107.7) (end 55.5 106.6) (width 1) (layer "F.Cu") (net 3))
 (segment (start 40.13 102.47) (end 41 101.6) (width 1) (layer "F.Cu") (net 3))
 (segment (start 30.1 137.7) (end 31.3 138.9) (width 1.5) (layer "F.Cu") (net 3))
 (segment (start 41 101.6) (end 41 94.9) (width 1) (layer "F.Cu") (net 3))
 (segment (start 28.03 105.6) (end 28 105.63) (width 1) (layer "F.Cu") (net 3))
 (segment (start 28.85 100.55) (end 32.3 97.1) (width 1) (layer "F.Cu") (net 19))
 (segment (start 32.3 97.1) (end 32.3 92.92) (width 1) (layer "F.Cu") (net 19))
 (segment (start 28 100.55) (end 28.85 100.55) (width 1) (layer "F.Cu") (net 19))
 (segment (start 71.26 134.92) (end 68.42 134.92) (width 1.5) (layer "F.Cu") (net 5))
 (segment (start 70.8 115) (end 72.9 117.1) (width 1.5) (layer "F.Cu") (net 5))
 (segment (start 72.9 117.1) (end 72.9 133.28) (width 1.5) (layer "F.Cu") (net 5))
 (segment (start 68.42 115) (end 70.8 115) (width 1.5) (layer "F.Cu") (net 5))
 (segment (start 68.42 115) (end 68.42 122.46) (width 1.5) (layer "F.Cu") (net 5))
 (segment (start 72.9 133.28) (end 71.26 134.92) (width 1.5) (layer "F.Cu") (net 5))
 (segment (start 53.28 100.1) (end 53.3 100.12) (width 1) (layer "F.Cu") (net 16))
 (segment (start 64.1 101.2) (end 65.6 102.7) (width 1) (layer "F.Cu") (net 16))
 (segment (start 62.6 96.7) (end 64.1 98.2) (width 1) (layer "F.Cu") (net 16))
 (segment (start 53.3 100.12) (end 56.5 100.12) (width 1) (layer "F.Cu") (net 16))
 (segment (start 56.5 100.12) (end 56.6 100.02) (width 1) (layer "F.Cu") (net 16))
 (segment (start 65.6 102.7) (end 65.62 102.68) (width 1) (layer "F.Cu") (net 16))
 (segment (start 56.6 100.02) (end 59.08 100.02) (width 1) (layer "F.Cu") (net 16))
 (segment (start 60.1 96.7) (end 62.6 96.7) (width 1) (layer "F.Cu") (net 16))
 (segment (start 59.08 100.02) (end 60.1 99) (width 1) (layer "F.Cu") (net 16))
 (segment (start 67.66 102.54) (end 68.3 101.9) (width 1) (layer "F.Cu") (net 16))
 (segment (start 68.2 102.8) (end 68.42 102.8) (width 1) (layer "F.Cu") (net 16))
 (segment (start 56.9 99.72) (end 56.6 100.02) (width 1) (layer "F.Cu") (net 16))
 (segment (start 65.62 102.68) (end 68.42 102.68) (width 1) (layer "F.Cu") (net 16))
 (segment (start 64.1 98.2) (end 64.1 101.2) (width 1) (layer "F.Cu") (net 16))
 (segment (start 60.1 99) (end 60.1 96.7) (width 1) (layer "F.Cu") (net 16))
 (segment (start 53.145 122.14) (end 47.54 122.14) (width 1.5) (layer "F.Cu") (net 11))
 (segment (start 39.9 116.1) (end 38.2 117.8) (width 1.5) (layer "F.Cu") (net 11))
 (segment (start 44.9 116.1) (end 39.9 116.1) (width 1.5) (layer "F.Cu") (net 11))
 (segment (start 47.54 122.14) (end 46.6 121.2) (width 1.5) (layer "F.Cu") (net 11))
 (segment (start 46.6 121.2) (end 46.6 117.8) (width 1.5) (layer "F.Cu") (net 11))
 (segment (start 46.6 117.8) (end 44.9 116.1) (width 1.5) (layer "F.Cu") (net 11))
 (segment (start 53.145 122.14) (end 53.17 122.115) (width 1) (layer "F.Cu") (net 11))
 (segment (start 38.2 117.8) (end 38.2 120.92) (width 1.5) (layer "F.Cu") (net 11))
 (segment (start 46.212439 96.7) (end 45.845 96.332561) (width 1) (layer "F.Cu") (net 1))
 (segment (start 55.34 93.787561) (end 52.427561 96.7) (width 1) (layer "F.Cu") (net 1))
 (segment (start 44.82 96.9) (end 44.72 96.8) (width 0.25) (layer "F.Cu") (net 1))
 (segment (start 45.02 96.9) (end 44.82 96.9) (width 0.25) (layer "F.Cu") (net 1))
 (segment (start 52.427561 96.7) (end 46.212439 96.7) (width 1) (layer "F.Cu") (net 1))
 (segment (start 60.11 93.787561) (end 55.34 93.787561) (width 1) (layer "F.Cu") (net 1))
 (segment (start 46.9 110.18) (end 50.1 110.18) (width 1) (layer "F.Cu") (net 14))
 (segment (start 53.2 110.18) (end 53.3 110.28) (width 1) (layer "F.Cu") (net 14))
 (segment (start 50.1 110.18) (end 53.2 110.18) (width 1) (layer "F.Cu") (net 14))
 (segment (start 41.5 133.72) (end 41.5 135.7) (width 1.2) (layer "F.Cu") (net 20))
 (segment (start 33.095 135.795) (end 33.095 134.165) (width 1.2) (layer "F.Cu") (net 20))
 (segment (start 41.5 135.7) (end 40.2 137) (width 1.2) (layer "F.Cu") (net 20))
 (segment (start 40.2 137) (end 34.3 137) (width 1.2) (layer "F.Cu") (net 20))
 (segment (start 34.3 137) (end 33.095 135.795) (width 1.2) (layer "F.Cu") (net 20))
 (segment (start 33.12 120.92) (end 33.12 123.16) (width 1.2) (layer "F.Cu") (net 13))
 (segment (start 34.62 124.66) (end 39.22 124.66) (width 1.2) (layer "F.Cu") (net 13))
 (segment (start 39.22 124.66) (end 41.4 122.48) (width 1.2) (layer "F.Cu") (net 13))
 (segment (start 41.4 122.48) (end 41.4 119.62) (width 1.2) (layer "F.Cu") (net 13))
 (segment (start 33.12 123.16) (end 34.62 124.66) (width 1.2) (layer "F.Cu") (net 13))
 (segment (start 27.8 139.1) (end 27.8 113.45) (width 1) (layer "F.Cu") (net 21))
 (segment (start 27.8 113.45) (end 28 113.25) (width 1) (layer "F.Cu") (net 21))
 (segment (start 30.485 141.785) (end 27.8 139.1) (width 1) (layer "F.Cu") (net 21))
 (segment (start 33.095 141.785) (end 30.485 141.785) (width 1) (layer "F.Cu") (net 21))
 (segment (start 32.3 128.54) (end 31.02 127.26) (width 1) (layer "F.Cu") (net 9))
 (segment (start 31.02 111.72) (end 30 110.7) (width 1) (layer "F.Cu") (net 9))
 (segment (start 33.12 128.54) (end 32.3 128.54) (width 1) (layer "F.Cu") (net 9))
 (segment (start 29.99 110.71) (end 28 110.71) (width 1) (layer "F.Cu") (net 9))
 (segment (start 31.02 127.26) (end 31.02 111.72) (width 1) (layer "F.Cu") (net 9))
 (segment (start 30 110.7) (end 29.99 110.71) (width 1) (layer "F.Cu") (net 9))
 (segment (start 38 105.01) (end 38 107.55) (width 1) (layer "F.Cu") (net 25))
 (segment (start 50.1 102.5) (end 50.1 100.02) (width 1) (layer "F.Cu") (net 25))
 (segment (start 58.3 103.8) (end 51.4 103.8) (width 1) (layer "F.Cu") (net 25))
 (segment (start 39.9 113) (end 58.2 113) (width 1) (layer "F.Cu") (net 25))
 (segment (start 58.2 113) (end 60.2 111) (width 1) (layer "F.Cu") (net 25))
 (segment (start 60.2 105.7) (end 58.3 103.8) (width 1) (layer "F.Cu") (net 25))
 (segment (start 60.2 111) (end 60.2 105.7) (width 1) (layer "F.Cu") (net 25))
 (segment (start 38 111.1) (end 39.9 113) (width 1) (layer "F.Cu") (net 25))
 (segment (start 37.38 108.17) (end 38 107.55) (width 1) (layer "F.Cu") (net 25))
 (segment (start 38 107.55) (end 38 111.1) (width 1) (layer "F.Cu") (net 25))
 (segment (start 51.4 103.8) (end 50.1 102.5) (width 1) (layer "F.Cu") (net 25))
 (segment (start 28 108.17) (end 37.38 108.17) (width 1) (layer "F.Cu") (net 25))
 (segment (start 32.29 103.09) (end 32.3 103.08) (width 1) (layer "F.Cu") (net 4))
 (segment (start 32.3 101.1) (end 37.067439 96.332561) (width 1) (layer "F.Cu") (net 4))
 (segment (start 37.067439 96.332561) (end 38.225 96.332561) (width 1) (layer "F.Cu") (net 4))
 (segment (start 32.3 103.08) (end 32.3 101.1) (width 1) (layer "F.Cu") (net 4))
 (segment (start 38.22 96.327561) (end 38.225 96.332561) (width 1) (layer "F.Cu") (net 4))
 (segment (start 28 103.09) (end 32.29 103.09) (width 1) (layer "F.Cu") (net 4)))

